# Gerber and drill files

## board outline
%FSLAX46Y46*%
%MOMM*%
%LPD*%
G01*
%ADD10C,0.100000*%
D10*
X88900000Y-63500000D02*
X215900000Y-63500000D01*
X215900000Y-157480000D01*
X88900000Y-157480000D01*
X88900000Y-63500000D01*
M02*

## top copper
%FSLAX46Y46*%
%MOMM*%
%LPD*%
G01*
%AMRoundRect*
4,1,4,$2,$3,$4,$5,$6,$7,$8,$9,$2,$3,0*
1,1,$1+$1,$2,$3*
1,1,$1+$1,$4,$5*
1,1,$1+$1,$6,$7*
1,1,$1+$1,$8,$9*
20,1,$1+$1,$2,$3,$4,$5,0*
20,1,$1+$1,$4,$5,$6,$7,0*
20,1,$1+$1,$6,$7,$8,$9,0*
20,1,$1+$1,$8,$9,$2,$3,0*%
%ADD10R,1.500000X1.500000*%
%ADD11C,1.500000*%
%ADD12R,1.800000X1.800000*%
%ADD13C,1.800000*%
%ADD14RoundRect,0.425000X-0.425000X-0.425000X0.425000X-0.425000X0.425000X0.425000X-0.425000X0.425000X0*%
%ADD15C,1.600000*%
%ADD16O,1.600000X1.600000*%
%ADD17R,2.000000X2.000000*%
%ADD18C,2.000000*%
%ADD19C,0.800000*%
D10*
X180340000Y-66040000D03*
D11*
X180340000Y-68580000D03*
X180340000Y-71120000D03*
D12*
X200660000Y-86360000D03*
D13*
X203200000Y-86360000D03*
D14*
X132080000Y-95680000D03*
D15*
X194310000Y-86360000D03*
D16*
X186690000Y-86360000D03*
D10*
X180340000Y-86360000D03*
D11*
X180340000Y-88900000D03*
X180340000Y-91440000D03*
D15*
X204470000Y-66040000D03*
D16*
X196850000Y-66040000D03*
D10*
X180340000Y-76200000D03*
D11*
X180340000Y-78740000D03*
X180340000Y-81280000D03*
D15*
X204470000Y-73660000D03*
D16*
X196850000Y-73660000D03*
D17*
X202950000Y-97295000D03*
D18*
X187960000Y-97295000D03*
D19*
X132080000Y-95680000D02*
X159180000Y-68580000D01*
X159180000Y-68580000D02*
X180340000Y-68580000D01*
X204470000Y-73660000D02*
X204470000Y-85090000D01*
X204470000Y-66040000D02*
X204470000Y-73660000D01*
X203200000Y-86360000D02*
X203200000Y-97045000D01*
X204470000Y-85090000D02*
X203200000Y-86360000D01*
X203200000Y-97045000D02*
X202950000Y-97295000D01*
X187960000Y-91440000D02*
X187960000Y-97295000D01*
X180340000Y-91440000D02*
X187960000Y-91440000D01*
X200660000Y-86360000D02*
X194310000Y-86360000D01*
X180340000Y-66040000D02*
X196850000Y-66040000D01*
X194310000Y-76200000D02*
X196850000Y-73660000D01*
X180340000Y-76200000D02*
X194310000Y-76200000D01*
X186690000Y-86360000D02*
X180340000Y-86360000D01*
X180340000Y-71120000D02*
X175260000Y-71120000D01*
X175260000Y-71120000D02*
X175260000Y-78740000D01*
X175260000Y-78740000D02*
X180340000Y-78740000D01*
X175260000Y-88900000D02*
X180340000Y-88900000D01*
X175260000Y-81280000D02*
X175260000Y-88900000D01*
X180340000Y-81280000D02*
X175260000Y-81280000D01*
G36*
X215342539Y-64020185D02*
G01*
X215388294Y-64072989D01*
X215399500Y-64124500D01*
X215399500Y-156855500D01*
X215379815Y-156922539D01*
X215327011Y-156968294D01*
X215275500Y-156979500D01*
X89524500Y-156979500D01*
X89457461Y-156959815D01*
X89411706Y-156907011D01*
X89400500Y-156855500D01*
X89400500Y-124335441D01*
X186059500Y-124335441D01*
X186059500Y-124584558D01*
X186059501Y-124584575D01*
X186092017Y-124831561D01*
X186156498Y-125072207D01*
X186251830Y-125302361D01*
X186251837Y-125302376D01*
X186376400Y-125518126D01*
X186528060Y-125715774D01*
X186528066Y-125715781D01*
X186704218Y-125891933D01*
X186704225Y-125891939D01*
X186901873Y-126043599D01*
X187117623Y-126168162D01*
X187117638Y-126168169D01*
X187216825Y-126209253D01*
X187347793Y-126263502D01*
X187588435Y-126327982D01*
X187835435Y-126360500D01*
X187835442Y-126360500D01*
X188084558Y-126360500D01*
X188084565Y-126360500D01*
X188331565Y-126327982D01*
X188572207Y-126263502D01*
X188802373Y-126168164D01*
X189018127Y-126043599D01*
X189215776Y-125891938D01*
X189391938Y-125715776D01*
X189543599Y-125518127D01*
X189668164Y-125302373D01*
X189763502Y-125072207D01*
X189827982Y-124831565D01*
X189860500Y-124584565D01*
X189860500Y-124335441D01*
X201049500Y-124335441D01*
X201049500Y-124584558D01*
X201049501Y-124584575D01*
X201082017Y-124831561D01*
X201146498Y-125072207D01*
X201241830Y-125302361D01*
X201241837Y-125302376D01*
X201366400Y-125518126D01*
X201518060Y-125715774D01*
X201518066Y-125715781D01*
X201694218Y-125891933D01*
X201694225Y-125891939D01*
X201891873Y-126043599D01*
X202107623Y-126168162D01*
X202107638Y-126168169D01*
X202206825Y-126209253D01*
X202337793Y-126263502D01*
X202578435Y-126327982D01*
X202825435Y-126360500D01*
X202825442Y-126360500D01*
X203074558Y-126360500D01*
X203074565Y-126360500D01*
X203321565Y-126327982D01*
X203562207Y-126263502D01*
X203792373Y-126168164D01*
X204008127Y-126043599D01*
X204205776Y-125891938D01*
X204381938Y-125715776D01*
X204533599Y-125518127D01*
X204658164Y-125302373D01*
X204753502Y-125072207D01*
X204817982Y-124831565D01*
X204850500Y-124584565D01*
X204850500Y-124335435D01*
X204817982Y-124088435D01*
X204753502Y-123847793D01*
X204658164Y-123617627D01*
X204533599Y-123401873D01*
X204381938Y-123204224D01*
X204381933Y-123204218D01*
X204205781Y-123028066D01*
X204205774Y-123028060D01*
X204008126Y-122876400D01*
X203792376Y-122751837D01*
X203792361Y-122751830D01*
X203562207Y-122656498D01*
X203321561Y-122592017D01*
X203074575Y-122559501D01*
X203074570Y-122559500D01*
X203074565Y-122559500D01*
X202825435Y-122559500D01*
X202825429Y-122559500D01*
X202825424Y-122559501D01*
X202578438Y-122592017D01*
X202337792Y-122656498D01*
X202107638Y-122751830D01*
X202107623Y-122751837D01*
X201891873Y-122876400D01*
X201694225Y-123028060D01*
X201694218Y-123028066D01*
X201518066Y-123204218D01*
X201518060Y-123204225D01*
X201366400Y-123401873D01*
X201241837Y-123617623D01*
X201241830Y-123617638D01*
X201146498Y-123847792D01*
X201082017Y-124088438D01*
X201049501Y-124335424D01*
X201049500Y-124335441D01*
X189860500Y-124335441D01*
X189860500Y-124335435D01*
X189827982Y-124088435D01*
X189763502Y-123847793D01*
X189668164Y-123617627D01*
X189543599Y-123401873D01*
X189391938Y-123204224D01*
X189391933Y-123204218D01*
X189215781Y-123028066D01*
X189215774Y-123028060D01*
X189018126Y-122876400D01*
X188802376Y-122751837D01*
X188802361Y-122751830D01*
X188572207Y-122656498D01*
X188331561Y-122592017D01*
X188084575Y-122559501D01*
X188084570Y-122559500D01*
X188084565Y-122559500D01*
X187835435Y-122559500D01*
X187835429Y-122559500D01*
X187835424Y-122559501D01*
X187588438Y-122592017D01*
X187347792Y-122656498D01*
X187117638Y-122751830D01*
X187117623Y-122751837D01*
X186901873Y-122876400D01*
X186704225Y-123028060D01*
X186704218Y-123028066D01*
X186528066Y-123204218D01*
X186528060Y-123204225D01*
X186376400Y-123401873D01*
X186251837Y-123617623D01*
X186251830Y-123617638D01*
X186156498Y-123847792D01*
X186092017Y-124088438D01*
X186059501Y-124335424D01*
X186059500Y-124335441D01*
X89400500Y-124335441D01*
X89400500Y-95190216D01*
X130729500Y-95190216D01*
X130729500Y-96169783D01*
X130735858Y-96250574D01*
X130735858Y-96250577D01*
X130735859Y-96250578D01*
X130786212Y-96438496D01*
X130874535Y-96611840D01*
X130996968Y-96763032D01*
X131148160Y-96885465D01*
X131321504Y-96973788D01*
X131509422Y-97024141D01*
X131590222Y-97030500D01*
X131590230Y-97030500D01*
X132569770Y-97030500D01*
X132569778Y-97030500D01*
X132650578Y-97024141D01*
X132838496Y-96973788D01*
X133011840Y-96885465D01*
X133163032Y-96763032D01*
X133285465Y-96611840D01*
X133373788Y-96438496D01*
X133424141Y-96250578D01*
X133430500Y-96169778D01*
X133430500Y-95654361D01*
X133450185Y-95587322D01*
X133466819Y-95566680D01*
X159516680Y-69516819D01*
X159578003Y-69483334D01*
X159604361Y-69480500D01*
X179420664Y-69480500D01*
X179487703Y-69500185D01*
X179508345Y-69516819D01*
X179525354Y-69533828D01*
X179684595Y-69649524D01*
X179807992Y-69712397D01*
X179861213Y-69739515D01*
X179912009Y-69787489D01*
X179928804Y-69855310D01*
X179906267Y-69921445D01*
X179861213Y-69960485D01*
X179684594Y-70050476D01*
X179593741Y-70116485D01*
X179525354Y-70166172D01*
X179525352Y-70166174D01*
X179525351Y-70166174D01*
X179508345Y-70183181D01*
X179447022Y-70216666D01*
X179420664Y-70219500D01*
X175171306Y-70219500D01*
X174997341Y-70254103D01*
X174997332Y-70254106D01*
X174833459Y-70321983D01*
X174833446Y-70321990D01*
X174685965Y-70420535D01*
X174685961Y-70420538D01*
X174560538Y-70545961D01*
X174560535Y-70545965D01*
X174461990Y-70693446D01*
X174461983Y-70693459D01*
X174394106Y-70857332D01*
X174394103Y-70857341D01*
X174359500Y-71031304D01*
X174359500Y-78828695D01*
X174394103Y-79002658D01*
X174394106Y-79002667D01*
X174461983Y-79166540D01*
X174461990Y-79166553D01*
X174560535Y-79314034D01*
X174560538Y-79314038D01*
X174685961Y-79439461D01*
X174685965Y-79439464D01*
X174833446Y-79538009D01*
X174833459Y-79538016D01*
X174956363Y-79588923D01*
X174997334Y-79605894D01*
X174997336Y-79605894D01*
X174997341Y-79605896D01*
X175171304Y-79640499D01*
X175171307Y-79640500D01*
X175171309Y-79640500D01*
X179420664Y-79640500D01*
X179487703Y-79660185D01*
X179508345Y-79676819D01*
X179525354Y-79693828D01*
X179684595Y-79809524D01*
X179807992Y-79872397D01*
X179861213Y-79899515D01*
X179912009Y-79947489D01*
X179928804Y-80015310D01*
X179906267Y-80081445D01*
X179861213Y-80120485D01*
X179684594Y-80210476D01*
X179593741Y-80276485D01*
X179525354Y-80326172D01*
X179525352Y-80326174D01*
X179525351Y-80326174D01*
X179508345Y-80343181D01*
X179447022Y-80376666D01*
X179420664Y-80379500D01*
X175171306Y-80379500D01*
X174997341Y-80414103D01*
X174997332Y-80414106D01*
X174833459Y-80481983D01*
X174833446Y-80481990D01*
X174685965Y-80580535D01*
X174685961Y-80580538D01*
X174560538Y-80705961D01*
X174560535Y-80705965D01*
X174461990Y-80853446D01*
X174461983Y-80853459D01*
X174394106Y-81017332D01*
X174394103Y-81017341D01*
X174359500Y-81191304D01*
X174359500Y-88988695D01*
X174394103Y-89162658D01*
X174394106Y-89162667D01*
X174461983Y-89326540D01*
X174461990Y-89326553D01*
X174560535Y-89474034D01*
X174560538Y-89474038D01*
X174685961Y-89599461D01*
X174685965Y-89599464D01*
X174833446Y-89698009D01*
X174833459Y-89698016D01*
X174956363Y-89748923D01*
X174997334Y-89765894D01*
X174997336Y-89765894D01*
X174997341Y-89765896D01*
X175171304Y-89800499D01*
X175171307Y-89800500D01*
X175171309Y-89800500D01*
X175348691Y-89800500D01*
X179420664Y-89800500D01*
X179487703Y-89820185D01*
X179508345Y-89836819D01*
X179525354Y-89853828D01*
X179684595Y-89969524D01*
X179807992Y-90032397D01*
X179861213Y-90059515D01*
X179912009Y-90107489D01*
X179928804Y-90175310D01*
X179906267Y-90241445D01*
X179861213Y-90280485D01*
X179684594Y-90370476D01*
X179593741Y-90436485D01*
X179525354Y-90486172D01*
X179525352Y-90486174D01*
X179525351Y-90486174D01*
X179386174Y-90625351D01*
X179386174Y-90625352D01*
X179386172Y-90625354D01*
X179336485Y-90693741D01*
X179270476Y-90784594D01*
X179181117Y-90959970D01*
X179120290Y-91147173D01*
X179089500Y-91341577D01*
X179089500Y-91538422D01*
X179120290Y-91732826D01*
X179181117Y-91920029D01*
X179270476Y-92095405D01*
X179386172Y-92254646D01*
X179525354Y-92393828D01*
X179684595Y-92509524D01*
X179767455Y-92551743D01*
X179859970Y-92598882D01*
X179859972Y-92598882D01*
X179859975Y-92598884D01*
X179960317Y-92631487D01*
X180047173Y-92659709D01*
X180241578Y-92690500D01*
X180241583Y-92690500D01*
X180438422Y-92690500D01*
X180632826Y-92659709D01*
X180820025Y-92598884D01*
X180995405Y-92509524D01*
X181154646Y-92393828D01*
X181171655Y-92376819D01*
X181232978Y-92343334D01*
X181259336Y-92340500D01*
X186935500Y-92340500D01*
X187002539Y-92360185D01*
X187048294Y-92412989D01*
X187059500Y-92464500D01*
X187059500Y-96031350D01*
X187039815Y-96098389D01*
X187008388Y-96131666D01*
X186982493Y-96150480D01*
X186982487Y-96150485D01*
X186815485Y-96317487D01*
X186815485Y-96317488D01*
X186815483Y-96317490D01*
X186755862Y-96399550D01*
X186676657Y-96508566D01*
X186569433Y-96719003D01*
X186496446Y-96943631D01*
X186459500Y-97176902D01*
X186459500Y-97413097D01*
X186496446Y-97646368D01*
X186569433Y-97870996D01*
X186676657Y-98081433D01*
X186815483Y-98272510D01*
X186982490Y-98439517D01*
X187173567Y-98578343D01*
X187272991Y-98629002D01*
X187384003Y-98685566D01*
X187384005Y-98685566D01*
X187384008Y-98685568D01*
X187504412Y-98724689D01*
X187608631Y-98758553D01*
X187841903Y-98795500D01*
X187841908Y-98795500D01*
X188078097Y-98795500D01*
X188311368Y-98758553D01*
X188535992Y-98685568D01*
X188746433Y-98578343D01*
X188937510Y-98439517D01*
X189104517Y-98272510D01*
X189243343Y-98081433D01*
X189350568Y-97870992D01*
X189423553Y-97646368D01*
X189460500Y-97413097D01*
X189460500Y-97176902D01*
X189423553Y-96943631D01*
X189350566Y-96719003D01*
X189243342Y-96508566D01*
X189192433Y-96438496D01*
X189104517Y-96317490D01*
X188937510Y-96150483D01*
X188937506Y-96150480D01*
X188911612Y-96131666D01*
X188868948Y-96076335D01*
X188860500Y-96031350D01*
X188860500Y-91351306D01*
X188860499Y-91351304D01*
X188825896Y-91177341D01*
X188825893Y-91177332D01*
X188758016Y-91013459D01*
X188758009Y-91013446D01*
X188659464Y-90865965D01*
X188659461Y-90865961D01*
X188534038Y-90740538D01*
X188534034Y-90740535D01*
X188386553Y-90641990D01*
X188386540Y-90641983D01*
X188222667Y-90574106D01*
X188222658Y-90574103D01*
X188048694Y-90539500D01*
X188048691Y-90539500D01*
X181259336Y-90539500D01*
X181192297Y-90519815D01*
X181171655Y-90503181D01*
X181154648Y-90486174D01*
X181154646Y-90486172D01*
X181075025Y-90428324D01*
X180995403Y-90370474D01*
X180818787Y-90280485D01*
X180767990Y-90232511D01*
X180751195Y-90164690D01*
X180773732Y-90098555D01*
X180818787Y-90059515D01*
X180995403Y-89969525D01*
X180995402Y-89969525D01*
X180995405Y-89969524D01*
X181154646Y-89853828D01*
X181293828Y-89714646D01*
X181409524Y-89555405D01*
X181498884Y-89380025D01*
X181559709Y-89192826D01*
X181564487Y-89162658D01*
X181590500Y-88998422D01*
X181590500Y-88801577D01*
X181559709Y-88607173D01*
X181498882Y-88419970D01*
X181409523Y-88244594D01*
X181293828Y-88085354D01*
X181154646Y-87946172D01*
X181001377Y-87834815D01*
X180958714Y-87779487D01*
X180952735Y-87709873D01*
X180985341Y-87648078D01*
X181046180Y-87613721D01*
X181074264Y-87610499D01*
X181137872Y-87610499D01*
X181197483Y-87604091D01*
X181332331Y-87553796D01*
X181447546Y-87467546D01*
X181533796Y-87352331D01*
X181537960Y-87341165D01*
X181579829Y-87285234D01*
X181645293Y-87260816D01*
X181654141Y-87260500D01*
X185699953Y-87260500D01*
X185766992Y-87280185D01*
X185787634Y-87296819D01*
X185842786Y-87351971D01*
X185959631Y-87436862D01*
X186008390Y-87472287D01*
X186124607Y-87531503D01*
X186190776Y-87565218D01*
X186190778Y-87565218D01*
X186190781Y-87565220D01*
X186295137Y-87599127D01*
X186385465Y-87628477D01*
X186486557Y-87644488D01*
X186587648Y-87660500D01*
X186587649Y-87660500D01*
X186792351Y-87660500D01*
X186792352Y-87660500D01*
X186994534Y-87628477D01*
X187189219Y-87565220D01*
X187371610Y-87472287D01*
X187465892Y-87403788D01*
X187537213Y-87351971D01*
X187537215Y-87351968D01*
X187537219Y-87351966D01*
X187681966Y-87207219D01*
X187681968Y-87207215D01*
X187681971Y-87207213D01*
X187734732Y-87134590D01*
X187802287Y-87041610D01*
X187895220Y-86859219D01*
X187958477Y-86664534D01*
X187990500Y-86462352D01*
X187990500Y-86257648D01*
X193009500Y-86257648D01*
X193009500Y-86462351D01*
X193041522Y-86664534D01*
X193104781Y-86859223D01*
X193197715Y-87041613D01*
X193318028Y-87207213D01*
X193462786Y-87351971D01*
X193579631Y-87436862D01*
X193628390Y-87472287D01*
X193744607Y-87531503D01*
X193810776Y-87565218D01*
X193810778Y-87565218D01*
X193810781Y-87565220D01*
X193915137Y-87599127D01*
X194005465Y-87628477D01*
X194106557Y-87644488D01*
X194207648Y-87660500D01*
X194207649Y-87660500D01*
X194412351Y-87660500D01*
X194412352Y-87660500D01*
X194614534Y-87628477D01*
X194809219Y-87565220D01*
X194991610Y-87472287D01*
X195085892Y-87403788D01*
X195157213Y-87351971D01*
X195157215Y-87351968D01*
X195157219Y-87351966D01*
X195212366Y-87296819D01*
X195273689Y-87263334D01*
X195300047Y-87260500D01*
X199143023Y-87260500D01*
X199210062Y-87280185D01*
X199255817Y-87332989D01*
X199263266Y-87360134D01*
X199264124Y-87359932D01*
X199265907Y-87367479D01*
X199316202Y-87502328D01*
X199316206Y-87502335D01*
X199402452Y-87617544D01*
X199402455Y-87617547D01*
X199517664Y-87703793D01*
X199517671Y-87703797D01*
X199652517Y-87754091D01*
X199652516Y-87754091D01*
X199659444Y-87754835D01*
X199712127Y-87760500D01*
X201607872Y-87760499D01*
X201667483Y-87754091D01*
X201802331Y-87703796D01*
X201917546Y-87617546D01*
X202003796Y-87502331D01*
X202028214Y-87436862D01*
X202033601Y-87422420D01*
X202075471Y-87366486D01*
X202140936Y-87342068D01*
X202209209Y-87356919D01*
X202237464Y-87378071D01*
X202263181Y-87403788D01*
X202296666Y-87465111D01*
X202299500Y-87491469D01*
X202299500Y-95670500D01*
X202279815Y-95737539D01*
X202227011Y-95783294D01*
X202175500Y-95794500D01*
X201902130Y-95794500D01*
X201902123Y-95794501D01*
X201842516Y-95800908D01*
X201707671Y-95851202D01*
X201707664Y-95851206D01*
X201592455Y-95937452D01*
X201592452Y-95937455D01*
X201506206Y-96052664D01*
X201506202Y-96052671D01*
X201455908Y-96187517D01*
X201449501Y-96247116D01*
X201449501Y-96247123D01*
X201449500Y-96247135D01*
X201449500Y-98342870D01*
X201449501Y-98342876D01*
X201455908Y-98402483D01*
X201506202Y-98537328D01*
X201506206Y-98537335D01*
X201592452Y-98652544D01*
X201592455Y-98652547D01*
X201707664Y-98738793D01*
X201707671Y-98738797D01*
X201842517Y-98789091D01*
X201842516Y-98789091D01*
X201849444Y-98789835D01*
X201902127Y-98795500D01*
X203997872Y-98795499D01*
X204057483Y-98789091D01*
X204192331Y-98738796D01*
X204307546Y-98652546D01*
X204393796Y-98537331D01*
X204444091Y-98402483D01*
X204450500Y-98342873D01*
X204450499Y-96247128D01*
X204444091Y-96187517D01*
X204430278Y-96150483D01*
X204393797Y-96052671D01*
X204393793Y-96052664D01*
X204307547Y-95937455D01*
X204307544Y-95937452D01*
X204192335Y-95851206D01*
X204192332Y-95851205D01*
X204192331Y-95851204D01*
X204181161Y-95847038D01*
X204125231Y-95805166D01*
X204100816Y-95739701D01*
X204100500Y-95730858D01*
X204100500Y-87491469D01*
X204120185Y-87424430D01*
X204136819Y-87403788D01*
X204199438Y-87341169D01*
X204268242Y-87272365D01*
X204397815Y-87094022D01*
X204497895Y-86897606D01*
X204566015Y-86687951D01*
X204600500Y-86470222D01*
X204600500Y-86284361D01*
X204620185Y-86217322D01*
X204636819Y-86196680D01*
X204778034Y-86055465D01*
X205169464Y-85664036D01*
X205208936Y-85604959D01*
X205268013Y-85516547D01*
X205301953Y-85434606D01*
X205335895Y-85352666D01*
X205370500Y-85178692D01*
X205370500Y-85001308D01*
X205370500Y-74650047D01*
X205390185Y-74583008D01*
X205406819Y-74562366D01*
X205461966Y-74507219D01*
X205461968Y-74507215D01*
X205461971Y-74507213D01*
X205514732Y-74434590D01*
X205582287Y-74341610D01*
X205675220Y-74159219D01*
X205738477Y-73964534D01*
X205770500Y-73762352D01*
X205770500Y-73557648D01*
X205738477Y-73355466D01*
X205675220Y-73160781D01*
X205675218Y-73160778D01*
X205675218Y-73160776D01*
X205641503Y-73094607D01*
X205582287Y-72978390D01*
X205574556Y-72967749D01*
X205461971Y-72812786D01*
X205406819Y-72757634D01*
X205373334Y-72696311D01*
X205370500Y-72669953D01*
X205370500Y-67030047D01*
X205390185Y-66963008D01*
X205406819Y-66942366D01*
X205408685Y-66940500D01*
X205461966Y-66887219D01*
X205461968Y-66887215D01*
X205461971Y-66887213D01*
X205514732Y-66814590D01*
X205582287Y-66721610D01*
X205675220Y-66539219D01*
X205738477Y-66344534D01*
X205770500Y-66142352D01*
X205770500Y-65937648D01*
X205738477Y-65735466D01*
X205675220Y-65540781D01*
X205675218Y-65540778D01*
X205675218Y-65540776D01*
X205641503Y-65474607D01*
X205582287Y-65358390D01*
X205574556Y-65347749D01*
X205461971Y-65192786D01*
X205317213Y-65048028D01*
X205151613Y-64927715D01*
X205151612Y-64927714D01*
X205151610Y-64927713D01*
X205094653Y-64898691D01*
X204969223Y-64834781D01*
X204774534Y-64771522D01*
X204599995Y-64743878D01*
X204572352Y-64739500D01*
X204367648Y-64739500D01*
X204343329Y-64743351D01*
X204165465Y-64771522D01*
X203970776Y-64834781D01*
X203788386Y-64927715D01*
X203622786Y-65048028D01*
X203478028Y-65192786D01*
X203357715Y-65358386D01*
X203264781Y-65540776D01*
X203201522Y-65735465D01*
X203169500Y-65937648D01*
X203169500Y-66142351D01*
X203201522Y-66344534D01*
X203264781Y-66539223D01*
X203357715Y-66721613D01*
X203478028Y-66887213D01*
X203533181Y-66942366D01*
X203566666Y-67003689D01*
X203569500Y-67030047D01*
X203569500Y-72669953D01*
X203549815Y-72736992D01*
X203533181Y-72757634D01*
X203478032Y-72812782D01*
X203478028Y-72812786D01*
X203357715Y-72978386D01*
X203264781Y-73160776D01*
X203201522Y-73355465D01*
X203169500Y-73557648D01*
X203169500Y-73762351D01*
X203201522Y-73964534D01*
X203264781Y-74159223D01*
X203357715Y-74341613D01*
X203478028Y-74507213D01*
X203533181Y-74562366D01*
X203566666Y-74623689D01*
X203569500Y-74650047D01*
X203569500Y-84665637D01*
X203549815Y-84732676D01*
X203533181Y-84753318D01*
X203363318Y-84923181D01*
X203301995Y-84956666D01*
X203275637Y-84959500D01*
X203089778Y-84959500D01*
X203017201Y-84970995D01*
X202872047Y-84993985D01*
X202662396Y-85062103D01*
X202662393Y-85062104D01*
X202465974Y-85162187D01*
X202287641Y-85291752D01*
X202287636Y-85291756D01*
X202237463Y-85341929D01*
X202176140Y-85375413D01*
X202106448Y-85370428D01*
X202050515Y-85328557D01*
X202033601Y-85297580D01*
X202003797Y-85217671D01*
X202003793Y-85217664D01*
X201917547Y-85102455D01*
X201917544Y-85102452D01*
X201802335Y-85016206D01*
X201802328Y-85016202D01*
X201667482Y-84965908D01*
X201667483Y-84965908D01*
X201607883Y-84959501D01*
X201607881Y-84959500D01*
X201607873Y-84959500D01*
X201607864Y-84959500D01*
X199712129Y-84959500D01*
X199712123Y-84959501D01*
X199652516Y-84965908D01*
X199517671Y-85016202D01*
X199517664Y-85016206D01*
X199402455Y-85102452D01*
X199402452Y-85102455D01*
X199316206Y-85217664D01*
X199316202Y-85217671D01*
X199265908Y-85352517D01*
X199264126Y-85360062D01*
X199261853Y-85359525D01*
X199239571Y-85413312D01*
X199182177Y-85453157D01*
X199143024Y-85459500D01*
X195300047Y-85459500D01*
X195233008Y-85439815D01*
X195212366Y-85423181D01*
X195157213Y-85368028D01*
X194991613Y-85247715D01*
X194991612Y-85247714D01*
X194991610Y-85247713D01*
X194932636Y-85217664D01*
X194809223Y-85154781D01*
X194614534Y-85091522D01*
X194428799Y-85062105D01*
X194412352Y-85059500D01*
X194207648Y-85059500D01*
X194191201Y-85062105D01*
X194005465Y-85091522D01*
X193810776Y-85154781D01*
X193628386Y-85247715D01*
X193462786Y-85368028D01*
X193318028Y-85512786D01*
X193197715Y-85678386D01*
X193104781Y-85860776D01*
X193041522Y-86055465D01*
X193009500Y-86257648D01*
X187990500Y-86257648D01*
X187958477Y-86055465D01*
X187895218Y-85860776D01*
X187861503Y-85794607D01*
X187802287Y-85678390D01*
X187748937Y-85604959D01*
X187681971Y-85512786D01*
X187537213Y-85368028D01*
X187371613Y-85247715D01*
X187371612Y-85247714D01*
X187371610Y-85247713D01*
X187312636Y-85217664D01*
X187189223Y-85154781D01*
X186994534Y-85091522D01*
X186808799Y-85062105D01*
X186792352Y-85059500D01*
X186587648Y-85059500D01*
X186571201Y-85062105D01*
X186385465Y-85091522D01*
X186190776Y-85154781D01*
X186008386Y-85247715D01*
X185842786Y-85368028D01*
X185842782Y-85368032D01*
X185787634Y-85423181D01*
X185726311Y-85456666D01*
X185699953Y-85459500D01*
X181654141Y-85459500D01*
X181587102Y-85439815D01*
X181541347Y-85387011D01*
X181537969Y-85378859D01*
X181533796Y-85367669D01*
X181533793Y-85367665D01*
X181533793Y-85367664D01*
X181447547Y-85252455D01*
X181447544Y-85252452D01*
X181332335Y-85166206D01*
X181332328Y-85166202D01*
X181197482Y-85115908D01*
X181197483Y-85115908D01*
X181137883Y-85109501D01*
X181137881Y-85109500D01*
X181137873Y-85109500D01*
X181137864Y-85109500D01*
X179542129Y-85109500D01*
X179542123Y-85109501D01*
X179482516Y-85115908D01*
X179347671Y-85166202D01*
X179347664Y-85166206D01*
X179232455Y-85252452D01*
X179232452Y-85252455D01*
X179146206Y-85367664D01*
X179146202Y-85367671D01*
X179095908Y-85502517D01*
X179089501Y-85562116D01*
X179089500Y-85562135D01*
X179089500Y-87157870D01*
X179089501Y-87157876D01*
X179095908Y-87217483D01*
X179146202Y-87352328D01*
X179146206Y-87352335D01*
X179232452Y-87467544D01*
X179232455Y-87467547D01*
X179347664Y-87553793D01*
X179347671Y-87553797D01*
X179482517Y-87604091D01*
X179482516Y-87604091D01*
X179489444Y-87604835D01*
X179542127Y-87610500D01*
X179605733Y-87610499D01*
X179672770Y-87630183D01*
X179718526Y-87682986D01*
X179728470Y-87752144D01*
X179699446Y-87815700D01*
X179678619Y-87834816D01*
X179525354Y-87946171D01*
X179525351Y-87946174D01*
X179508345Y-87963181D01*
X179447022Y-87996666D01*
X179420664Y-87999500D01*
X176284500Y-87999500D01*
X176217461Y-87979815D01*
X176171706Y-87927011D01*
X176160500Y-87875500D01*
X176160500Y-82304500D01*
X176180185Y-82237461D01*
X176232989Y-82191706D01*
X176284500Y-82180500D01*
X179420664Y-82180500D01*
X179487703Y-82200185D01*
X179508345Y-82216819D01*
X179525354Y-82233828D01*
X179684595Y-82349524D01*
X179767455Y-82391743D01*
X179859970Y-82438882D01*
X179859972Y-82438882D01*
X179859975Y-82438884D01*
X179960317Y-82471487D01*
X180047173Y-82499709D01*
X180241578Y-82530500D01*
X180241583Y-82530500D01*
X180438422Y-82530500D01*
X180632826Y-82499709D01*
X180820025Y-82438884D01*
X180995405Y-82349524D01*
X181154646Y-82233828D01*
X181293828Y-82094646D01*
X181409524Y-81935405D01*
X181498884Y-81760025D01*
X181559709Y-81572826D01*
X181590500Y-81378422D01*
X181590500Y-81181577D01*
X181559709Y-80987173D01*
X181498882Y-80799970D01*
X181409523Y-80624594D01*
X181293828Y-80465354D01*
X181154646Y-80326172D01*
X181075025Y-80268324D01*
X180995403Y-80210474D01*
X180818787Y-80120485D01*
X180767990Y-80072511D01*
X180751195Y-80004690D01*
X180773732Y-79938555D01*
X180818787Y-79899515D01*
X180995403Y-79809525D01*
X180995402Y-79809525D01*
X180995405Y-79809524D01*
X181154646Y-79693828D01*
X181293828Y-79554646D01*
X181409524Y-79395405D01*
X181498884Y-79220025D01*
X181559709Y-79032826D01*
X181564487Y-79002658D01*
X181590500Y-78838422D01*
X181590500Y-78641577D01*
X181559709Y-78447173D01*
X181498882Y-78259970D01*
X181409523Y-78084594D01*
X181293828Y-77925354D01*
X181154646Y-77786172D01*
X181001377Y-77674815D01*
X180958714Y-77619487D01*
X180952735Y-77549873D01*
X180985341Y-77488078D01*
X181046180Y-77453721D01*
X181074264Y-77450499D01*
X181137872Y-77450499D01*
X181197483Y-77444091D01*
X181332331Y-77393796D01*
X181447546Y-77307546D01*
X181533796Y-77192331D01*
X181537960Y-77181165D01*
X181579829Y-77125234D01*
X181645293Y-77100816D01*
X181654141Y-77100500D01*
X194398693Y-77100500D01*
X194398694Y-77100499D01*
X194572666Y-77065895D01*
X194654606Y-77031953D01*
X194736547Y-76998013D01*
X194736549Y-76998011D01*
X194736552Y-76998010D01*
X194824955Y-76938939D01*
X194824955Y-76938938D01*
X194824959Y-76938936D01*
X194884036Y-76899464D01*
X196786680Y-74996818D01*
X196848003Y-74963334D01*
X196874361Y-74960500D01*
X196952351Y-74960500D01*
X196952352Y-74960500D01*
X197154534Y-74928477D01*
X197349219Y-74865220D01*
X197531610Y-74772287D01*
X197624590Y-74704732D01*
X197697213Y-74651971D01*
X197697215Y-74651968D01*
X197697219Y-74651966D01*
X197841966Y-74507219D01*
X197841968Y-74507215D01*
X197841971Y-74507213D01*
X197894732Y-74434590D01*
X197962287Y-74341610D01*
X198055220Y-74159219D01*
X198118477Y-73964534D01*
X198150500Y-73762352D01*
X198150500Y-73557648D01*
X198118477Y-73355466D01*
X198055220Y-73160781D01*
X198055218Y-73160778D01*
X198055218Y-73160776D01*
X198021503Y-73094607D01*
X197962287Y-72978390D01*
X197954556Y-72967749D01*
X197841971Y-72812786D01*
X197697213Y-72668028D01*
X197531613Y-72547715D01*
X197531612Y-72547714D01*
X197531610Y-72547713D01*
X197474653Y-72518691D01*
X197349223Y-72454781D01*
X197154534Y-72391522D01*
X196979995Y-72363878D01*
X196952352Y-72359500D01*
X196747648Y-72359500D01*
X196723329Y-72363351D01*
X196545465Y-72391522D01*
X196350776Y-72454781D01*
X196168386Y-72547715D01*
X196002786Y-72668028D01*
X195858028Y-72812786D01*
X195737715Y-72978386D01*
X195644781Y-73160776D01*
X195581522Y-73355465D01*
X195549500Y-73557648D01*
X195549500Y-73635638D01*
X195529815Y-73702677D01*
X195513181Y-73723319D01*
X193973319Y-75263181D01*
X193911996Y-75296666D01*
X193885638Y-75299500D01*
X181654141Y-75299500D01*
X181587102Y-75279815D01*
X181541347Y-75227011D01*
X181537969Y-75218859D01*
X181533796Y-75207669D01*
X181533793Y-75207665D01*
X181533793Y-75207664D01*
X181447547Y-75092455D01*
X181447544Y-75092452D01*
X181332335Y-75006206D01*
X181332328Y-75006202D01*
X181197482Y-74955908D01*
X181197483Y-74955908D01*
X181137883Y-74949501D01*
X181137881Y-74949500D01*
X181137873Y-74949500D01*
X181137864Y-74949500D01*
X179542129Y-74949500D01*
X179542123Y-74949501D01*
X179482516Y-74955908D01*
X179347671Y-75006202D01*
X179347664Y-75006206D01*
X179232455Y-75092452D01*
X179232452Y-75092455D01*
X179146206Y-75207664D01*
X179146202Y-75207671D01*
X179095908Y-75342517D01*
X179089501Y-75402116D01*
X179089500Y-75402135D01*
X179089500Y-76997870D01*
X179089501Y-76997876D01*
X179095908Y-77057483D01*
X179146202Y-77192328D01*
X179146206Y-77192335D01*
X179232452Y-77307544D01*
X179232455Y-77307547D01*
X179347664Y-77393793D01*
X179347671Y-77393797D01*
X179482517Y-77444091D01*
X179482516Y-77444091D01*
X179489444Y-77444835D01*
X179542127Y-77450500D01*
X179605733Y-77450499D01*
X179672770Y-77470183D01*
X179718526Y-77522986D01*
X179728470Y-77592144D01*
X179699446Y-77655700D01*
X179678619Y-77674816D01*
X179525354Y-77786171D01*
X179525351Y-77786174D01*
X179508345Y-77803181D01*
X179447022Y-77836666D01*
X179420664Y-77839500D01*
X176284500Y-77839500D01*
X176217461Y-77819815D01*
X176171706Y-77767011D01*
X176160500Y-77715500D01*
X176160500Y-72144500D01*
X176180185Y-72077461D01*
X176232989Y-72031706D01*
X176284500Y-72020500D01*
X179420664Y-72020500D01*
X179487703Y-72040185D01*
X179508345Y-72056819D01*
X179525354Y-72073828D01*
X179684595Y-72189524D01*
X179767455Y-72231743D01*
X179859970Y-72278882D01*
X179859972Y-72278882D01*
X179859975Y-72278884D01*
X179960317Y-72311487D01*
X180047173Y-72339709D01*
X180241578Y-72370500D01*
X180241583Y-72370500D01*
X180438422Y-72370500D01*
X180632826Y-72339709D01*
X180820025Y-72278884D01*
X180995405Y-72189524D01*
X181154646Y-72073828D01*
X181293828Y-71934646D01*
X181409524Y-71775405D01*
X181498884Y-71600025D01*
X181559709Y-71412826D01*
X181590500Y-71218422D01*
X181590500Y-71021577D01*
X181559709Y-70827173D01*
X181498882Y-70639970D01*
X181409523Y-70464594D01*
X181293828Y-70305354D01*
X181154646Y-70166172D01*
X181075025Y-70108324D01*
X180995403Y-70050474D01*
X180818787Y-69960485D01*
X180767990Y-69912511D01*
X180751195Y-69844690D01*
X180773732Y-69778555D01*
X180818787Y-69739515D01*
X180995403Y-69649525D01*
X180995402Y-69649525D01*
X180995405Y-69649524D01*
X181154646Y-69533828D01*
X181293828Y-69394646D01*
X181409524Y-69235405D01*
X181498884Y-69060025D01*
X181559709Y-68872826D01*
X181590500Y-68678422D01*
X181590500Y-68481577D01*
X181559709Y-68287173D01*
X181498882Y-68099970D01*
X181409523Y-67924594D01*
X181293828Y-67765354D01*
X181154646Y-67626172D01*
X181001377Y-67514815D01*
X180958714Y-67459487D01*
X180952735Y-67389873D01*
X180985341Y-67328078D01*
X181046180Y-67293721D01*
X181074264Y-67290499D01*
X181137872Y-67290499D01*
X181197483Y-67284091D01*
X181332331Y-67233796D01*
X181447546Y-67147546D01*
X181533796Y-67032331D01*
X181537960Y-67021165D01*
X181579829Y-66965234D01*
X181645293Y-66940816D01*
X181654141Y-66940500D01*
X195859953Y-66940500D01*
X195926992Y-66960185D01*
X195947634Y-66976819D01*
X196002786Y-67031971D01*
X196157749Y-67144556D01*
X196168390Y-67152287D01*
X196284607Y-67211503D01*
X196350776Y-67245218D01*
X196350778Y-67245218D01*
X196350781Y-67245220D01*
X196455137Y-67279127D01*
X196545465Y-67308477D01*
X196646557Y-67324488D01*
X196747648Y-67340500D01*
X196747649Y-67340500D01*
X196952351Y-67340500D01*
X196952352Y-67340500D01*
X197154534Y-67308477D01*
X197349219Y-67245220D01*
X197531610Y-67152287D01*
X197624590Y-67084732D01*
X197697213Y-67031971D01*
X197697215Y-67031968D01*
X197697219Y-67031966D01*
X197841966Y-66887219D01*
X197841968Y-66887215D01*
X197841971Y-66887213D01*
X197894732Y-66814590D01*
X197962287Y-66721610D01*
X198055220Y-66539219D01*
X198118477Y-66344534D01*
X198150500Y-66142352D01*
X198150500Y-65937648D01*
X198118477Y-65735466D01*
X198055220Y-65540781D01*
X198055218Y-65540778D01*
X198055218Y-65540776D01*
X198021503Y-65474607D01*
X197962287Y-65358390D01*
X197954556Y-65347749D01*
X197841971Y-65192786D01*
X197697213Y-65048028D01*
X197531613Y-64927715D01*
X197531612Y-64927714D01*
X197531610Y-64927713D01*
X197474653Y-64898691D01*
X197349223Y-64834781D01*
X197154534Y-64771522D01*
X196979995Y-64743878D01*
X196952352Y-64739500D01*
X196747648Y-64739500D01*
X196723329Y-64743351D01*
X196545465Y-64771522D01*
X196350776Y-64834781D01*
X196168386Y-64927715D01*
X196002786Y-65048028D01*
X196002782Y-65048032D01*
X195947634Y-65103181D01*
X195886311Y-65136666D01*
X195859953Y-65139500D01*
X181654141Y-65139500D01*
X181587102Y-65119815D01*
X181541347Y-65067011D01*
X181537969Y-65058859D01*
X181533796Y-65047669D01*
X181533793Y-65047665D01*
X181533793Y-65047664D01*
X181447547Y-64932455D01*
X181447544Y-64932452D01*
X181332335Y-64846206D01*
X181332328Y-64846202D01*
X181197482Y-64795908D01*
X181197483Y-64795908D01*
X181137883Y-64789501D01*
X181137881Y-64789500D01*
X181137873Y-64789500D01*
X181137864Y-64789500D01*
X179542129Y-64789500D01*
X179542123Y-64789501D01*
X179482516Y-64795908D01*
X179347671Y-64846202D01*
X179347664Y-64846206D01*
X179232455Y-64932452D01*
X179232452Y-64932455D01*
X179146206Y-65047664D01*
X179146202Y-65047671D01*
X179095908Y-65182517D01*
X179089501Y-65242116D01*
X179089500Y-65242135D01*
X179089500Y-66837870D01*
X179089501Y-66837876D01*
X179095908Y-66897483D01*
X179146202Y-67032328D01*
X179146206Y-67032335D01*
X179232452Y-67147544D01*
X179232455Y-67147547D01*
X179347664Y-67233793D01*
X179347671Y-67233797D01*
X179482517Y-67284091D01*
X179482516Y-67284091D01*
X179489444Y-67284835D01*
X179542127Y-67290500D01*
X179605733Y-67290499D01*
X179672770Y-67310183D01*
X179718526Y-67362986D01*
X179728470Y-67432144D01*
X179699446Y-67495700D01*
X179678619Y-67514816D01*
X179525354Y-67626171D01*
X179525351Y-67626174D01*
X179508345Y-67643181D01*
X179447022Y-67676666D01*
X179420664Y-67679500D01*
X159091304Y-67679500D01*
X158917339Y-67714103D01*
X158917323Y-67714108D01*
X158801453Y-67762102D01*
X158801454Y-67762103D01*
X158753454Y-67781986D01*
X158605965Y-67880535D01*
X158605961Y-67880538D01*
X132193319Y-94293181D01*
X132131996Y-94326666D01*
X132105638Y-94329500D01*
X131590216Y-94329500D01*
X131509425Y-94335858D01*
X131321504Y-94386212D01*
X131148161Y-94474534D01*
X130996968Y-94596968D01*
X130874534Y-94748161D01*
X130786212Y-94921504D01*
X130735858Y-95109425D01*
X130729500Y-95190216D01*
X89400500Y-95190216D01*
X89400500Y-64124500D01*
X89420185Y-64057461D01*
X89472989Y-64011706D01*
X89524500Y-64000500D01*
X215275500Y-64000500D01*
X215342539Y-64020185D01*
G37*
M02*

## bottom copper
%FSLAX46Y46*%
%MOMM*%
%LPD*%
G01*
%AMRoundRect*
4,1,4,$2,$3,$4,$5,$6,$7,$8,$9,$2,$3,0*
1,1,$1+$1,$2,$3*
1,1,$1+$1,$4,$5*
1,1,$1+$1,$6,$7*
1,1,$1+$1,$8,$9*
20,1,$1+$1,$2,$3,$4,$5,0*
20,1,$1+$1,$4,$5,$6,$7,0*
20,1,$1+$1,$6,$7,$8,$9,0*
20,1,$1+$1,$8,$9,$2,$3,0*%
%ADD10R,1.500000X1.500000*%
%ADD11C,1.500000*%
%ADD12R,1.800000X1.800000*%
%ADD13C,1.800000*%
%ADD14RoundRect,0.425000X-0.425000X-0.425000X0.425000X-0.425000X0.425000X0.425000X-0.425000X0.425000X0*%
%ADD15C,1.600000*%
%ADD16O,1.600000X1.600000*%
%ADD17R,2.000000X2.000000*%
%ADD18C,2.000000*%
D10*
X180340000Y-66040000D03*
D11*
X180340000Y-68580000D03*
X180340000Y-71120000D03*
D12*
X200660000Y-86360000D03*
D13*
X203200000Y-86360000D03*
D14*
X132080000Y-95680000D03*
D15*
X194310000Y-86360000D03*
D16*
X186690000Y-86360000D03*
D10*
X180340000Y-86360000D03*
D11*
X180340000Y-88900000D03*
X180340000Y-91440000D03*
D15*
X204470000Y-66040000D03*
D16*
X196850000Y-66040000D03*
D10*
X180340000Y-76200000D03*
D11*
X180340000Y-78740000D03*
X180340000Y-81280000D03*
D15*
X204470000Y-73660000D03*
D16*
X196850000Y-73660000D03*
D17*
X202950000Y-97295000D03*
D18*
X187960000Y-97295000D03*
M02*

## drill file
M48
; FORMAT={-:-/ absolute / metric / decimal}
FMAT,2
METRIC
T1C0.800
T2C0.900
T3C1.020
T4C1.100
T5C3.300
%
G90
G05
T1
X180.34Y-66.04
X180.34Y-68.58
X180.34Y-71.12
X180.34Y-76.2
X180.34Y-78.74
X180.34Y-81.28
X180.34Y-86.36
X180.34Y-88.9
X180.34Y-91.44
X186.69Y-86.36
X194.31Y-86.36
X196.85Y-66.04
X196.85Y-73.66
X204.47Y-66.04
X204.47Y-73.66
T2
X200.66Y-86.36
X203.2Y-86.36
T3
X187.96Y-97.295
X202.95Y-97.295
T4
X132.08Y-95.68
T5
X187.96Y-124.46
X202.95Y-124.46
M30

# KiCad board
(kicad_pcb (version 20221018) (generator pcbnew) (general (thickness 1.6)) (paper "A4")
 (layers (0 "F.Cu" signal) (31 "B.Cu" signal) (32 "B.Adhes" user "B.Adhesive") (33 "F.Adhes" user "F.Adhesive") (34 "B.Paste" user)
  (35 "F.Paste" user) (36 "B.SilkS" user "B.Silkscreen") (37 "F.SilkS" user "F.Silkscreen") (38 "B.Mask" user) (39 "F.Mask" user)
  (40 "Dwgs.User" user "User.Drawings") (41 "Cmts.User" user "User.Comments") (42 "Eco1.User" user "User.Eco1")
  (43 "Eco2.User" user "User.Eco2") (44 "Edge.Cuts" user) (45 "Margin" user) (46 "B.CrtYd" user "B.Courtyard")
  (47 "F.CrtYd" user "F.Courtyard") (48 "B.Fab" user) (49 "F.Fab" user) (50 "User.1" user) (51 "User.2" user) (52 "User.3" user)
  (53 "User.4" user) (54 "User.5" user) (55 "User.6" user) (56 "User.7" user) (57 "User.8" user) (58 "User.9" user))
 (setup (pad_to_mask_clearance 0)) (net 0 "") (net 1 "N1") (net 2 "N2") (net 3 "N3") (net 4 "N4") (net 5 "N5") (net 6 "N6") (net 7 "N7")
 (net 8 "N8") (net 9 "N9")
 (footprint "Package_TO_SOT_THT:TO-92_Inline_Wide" (layer "F.Cu") (at 180.34 66.04 -90)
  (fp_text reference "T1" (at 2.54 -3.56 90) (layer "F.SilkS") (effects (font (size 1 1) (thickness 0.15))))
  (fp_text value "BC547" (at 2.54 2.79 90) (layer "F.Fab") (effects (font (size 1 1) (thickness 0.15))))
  (pad "1" thru_hole rect (at 0 0 270) (size 1.5 1.5) (drill 0.8) (layers "*.Cu" "*.Mask") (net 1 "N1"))
  (pad "2" thru_hole circle (at 2.54 0 270) (size 1.5 1.5) (drill 0.8) (layers "*.Cu" "*.Mask") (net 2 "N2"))
  (pad "3" thru_hole circle (at 5.08 0 270) (size 1.5 1.5) (drill 0.8) (layers "*.Cu" "*.Mask") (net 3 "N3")))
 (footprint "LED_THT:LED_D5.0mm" (layer "F.Cu") (at 200.66 86.36)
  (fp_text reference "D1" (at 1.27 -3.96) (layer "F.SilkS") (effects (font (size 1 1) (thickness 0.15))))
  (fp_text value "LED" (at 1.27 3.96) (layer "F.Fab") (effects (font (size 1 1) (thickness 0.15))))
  (pad "1" thru_hole rect (at 0 0) (size 1.8 1.8) (drill 0.9) (layers "*.Cu" "*.Mask") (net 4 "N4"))
  (pad "2" thru_hole circle (at 2.54 0) (size 1.8 1.8) (drill 0.9) (layers "*.Cu" "*.Mask") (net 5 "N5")))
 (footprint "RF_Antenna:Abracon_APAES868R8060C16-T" (layer "F.Cu") (at 132.08 95.68)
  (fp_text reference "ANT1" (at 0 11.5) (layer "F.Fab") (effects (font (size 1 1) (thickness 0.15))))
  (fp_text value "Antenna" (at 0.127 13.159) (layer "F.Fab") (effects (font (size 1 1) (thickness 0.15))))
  (pad "1" thru_hole roundrect (at 0 0) (size 1.7 1.7) (drill 1.1) (layers "*.Cu" "*.Mask") (roundrect_rratio 0.25) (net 2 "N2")))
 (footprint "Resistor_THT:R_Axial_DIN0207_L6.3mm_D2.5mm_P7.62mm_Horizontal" (layer "F.Cu") (at 194.31 86.36 180)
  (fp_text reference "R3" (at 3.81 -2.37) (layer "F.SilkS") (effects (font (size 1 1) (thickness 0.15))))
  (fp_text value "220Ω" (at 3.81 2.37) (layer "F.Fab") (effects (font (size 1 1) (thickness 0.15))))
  (pad "1" thru_hole circle (at 0 0 180) (size 1.6 1.6) (drill 0.8) (layers "*.Cu" "*.Mask") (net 4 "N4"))
  (pad "2" thru_hole oval (at 7.62 0 180) (size 1.6 1.6) (drill 0.8) (layers "*.Cu" "*.Mask") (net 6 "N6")))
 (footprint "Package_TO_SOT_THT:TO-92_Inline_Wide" (layer "F.Cu") (at 180.34 86.36 -90)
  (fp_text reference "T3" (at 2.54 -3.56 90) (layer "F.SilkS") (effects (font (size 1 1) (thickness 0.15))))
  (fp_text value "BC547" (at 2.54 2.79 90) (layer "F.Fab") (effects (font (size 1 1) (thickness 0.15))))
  (pad "1" thru_hole rect (at 0 0 270) (size 1.5 1.5) (drill 0.8) (layers "*.Cu" "*.Mask") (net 6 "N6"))
  (pad "2" thru_hole circle (at 2.54 0 270) (size 1.5 1.5) (drill 0.8) (layers "*.Cu" "*.Mask") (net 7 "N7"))
  (pad "3" thru_hole circle (at 5.08 0 270) (size 1.5 1.5) (drill 0.8) (layers "*.Cu" "*.Mask") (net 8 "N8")))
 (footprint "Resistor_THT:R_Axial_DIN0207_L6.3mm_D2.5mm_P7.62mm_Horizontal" (layer "F.Cu") (at 204.47 66.04 180)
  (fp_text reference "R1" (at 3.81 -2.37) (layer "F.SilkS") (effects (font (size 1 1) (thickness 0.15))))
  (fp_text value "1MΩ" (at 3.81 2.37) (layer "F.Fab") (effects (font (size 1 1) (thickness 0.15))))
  (pad "1" thru_hole circle (at 0 0 180) (size 1.6 1.6) (drill 0.8) (layers "*.Cu" "*.Mask") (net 5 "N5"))
  (pad "2" thru_hole oval (at 7.62 0 180) (size 1.6 1.6) (drill 0.8) (layers "*.Cu" "*.Mask") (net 1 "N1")))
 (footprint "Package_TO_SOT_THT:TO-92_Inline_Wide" (layer "F.Cu") (at 180.34 76.2 -90)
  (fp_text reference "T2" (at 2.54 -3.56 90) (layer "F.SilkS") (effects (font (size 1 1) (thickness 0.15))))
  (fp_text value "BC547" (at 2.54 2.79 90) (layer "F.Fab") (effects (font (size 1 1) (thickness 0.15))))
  (pad "1" thru_hole rect (at 0 0 270) (size 1.5 1.5) (drill 0.8) (layers "*.Cu" "*.Mask") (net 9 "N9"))
  (pad "2" thru_hole circle (at 2.54 0 270) (size 1.5 1.5) (drill 0.8) (layers "*.Cu" "*.Mask") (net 3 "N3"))
  (pad "3" thru_hole circle (at 5.08 0 270) (size 1.5 1.5) (drill 0.8) (layers "*.Cu" "*.Mask") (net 7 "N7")))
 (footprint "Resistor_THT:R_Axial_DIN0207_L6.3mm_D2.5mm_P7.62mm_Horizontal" (layer "F.Cu") (at 204.47 73.66 180)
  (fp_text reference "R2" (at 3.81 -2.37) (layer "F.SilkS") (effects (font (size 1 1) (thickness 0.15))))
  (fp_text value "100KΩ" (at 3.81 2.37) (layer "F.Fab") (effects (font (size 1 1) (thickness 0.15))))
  (pad "1" thru_hole circle (at 0 0 180) (size 1.6 1.6) (drill 0.8) (layers "*.Cu" "*.Mask") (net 5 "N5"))
  (pad "2" thru_hole oval (at 7.62 0 180) (size 1.6 1.6) (drill 0.8) (layers "*.Cu" "*.Mask") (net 9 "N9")))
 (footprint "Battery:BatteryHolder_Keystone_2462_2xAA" (layer "F.Cu") (at 202.95 97.295 -90)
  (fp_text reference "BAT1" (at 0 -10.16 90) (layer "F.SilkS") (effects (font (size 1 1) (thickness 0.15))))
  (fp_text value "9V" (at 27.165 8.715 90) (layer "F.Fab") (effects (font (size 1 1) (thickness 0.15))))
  (pad "" np_thru_hole circle (at 27.165 0 270) (size 3.3 3.3) (drill 3.3) (layers "*.Cu" "*.Mask"))
  (pad "" np_thru_hole circle (at 27.165 14.99 270) (size 3.3 3.3) (drill 3.3) (layers "*.Cu" "*.Mask"))
  (pad "1" thru_hole rect (at 0 0 270) (size 2 2) (drill 1.02) (layers "*.Cu" "*.Mask") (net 5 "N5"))
  (pad "2" thru_hole circle (at 0 14.99 270) (size 2 2) (drill 1.02) (layers "*.Cu" "*.Mask") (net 8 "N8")))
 (gr_rect (start 88.9 63.5) (end 215.9 157.48) (stroke (width 0.1) (type default)) (fill none) (layer "Edge.Cuts"))
 (segment (start 132.08 95.68) (end 159.18 68.58) (width 0.8) (layer "F.Cu") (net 2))
 (segment (start 159.18 68.58) (end 180.34 68.58) (width 0.8) (layer "F.Cu") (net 2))
 (segment (start 204.47 73.66) (end 204.47 85.09) (width 0.8) (layer "F.Cu") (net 5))
 (segment (start 204.47 66.04) (end 204.47 73.66) (width 0.8) (layer "F.Cu") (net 5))
 (segment (start 203.2 86.36) (end 203.2 97.045) (width 0.8) (layer "F.Cu") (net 5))
 (segment (start 204.47 85.09) (end 203.2 86.36) (width 0.8) (layer "F.Cu") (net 5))
 (segment (start 203.2 97.045) (end 202.95 97.295) (width 0.8) (layer "F.Cu") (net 5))
 (segment (start 187.96 91.44) (end 187.96 97.295) (width 0.8) (layer "F.Cu") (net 8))
 (segment (start 180.34 91.44) (end 187.96 91.44) (width 0.8) (layer "F.Cu") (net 8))
 (segment (start 200.66 86.36) (end 194.31 86.36) (width 0.8) (layer "F.Cu") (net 4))
 (segment (start 180.34 66.04) (end 196.85 66.04) (width 0.8) (layer "F.Cu") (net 1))
 (segment (start 194.31 76.2) (end 196.85 73.66) (width 0.8) (layer "F.Cu") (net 9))
 (segment (start 180.34 76.2) (end 194.31 76.2) (width 0.8) (layer "F.Cu") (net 9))
 (segment (start 186.69 86.36) (end 180.34 86.36) (width 0.8) (layer "F.Cu") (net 6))
 (segment (start 180.34 71.12) (end 175.26 71.12) (width 0.8) (layer "F.Cu") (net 3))
 (segment (start 175.26 71.12) (end 175.26 78.74) (width 0.8) (layer "F.Cu") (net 3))
 (segment (start 175.26 78.74) (end 180.34 78.74) (width 0.8) (layer "F.Cu") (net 3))
 (segment (start 175.26 88.9) (end 180.34 88.9) (width 0.8) (layer "F.Cu") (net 7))
 (segment (start 175.26 81.28) (end 175.26 88.9) (width 0.8) (layer "F.Cu") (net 7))
 (segment (start 180.34 81.28) (end 175.26 81.28) (width 0.8) (layer "F.Cu") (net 7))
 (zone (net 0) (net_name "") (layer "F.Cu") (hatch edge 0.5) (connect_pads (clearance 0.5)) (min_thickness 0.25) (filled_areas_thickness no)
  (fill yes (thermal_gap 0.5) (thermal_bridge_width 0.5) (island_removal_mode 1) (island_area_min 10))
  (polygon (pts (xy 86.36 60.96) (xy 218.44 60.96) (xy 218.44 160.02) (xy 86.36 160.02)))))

